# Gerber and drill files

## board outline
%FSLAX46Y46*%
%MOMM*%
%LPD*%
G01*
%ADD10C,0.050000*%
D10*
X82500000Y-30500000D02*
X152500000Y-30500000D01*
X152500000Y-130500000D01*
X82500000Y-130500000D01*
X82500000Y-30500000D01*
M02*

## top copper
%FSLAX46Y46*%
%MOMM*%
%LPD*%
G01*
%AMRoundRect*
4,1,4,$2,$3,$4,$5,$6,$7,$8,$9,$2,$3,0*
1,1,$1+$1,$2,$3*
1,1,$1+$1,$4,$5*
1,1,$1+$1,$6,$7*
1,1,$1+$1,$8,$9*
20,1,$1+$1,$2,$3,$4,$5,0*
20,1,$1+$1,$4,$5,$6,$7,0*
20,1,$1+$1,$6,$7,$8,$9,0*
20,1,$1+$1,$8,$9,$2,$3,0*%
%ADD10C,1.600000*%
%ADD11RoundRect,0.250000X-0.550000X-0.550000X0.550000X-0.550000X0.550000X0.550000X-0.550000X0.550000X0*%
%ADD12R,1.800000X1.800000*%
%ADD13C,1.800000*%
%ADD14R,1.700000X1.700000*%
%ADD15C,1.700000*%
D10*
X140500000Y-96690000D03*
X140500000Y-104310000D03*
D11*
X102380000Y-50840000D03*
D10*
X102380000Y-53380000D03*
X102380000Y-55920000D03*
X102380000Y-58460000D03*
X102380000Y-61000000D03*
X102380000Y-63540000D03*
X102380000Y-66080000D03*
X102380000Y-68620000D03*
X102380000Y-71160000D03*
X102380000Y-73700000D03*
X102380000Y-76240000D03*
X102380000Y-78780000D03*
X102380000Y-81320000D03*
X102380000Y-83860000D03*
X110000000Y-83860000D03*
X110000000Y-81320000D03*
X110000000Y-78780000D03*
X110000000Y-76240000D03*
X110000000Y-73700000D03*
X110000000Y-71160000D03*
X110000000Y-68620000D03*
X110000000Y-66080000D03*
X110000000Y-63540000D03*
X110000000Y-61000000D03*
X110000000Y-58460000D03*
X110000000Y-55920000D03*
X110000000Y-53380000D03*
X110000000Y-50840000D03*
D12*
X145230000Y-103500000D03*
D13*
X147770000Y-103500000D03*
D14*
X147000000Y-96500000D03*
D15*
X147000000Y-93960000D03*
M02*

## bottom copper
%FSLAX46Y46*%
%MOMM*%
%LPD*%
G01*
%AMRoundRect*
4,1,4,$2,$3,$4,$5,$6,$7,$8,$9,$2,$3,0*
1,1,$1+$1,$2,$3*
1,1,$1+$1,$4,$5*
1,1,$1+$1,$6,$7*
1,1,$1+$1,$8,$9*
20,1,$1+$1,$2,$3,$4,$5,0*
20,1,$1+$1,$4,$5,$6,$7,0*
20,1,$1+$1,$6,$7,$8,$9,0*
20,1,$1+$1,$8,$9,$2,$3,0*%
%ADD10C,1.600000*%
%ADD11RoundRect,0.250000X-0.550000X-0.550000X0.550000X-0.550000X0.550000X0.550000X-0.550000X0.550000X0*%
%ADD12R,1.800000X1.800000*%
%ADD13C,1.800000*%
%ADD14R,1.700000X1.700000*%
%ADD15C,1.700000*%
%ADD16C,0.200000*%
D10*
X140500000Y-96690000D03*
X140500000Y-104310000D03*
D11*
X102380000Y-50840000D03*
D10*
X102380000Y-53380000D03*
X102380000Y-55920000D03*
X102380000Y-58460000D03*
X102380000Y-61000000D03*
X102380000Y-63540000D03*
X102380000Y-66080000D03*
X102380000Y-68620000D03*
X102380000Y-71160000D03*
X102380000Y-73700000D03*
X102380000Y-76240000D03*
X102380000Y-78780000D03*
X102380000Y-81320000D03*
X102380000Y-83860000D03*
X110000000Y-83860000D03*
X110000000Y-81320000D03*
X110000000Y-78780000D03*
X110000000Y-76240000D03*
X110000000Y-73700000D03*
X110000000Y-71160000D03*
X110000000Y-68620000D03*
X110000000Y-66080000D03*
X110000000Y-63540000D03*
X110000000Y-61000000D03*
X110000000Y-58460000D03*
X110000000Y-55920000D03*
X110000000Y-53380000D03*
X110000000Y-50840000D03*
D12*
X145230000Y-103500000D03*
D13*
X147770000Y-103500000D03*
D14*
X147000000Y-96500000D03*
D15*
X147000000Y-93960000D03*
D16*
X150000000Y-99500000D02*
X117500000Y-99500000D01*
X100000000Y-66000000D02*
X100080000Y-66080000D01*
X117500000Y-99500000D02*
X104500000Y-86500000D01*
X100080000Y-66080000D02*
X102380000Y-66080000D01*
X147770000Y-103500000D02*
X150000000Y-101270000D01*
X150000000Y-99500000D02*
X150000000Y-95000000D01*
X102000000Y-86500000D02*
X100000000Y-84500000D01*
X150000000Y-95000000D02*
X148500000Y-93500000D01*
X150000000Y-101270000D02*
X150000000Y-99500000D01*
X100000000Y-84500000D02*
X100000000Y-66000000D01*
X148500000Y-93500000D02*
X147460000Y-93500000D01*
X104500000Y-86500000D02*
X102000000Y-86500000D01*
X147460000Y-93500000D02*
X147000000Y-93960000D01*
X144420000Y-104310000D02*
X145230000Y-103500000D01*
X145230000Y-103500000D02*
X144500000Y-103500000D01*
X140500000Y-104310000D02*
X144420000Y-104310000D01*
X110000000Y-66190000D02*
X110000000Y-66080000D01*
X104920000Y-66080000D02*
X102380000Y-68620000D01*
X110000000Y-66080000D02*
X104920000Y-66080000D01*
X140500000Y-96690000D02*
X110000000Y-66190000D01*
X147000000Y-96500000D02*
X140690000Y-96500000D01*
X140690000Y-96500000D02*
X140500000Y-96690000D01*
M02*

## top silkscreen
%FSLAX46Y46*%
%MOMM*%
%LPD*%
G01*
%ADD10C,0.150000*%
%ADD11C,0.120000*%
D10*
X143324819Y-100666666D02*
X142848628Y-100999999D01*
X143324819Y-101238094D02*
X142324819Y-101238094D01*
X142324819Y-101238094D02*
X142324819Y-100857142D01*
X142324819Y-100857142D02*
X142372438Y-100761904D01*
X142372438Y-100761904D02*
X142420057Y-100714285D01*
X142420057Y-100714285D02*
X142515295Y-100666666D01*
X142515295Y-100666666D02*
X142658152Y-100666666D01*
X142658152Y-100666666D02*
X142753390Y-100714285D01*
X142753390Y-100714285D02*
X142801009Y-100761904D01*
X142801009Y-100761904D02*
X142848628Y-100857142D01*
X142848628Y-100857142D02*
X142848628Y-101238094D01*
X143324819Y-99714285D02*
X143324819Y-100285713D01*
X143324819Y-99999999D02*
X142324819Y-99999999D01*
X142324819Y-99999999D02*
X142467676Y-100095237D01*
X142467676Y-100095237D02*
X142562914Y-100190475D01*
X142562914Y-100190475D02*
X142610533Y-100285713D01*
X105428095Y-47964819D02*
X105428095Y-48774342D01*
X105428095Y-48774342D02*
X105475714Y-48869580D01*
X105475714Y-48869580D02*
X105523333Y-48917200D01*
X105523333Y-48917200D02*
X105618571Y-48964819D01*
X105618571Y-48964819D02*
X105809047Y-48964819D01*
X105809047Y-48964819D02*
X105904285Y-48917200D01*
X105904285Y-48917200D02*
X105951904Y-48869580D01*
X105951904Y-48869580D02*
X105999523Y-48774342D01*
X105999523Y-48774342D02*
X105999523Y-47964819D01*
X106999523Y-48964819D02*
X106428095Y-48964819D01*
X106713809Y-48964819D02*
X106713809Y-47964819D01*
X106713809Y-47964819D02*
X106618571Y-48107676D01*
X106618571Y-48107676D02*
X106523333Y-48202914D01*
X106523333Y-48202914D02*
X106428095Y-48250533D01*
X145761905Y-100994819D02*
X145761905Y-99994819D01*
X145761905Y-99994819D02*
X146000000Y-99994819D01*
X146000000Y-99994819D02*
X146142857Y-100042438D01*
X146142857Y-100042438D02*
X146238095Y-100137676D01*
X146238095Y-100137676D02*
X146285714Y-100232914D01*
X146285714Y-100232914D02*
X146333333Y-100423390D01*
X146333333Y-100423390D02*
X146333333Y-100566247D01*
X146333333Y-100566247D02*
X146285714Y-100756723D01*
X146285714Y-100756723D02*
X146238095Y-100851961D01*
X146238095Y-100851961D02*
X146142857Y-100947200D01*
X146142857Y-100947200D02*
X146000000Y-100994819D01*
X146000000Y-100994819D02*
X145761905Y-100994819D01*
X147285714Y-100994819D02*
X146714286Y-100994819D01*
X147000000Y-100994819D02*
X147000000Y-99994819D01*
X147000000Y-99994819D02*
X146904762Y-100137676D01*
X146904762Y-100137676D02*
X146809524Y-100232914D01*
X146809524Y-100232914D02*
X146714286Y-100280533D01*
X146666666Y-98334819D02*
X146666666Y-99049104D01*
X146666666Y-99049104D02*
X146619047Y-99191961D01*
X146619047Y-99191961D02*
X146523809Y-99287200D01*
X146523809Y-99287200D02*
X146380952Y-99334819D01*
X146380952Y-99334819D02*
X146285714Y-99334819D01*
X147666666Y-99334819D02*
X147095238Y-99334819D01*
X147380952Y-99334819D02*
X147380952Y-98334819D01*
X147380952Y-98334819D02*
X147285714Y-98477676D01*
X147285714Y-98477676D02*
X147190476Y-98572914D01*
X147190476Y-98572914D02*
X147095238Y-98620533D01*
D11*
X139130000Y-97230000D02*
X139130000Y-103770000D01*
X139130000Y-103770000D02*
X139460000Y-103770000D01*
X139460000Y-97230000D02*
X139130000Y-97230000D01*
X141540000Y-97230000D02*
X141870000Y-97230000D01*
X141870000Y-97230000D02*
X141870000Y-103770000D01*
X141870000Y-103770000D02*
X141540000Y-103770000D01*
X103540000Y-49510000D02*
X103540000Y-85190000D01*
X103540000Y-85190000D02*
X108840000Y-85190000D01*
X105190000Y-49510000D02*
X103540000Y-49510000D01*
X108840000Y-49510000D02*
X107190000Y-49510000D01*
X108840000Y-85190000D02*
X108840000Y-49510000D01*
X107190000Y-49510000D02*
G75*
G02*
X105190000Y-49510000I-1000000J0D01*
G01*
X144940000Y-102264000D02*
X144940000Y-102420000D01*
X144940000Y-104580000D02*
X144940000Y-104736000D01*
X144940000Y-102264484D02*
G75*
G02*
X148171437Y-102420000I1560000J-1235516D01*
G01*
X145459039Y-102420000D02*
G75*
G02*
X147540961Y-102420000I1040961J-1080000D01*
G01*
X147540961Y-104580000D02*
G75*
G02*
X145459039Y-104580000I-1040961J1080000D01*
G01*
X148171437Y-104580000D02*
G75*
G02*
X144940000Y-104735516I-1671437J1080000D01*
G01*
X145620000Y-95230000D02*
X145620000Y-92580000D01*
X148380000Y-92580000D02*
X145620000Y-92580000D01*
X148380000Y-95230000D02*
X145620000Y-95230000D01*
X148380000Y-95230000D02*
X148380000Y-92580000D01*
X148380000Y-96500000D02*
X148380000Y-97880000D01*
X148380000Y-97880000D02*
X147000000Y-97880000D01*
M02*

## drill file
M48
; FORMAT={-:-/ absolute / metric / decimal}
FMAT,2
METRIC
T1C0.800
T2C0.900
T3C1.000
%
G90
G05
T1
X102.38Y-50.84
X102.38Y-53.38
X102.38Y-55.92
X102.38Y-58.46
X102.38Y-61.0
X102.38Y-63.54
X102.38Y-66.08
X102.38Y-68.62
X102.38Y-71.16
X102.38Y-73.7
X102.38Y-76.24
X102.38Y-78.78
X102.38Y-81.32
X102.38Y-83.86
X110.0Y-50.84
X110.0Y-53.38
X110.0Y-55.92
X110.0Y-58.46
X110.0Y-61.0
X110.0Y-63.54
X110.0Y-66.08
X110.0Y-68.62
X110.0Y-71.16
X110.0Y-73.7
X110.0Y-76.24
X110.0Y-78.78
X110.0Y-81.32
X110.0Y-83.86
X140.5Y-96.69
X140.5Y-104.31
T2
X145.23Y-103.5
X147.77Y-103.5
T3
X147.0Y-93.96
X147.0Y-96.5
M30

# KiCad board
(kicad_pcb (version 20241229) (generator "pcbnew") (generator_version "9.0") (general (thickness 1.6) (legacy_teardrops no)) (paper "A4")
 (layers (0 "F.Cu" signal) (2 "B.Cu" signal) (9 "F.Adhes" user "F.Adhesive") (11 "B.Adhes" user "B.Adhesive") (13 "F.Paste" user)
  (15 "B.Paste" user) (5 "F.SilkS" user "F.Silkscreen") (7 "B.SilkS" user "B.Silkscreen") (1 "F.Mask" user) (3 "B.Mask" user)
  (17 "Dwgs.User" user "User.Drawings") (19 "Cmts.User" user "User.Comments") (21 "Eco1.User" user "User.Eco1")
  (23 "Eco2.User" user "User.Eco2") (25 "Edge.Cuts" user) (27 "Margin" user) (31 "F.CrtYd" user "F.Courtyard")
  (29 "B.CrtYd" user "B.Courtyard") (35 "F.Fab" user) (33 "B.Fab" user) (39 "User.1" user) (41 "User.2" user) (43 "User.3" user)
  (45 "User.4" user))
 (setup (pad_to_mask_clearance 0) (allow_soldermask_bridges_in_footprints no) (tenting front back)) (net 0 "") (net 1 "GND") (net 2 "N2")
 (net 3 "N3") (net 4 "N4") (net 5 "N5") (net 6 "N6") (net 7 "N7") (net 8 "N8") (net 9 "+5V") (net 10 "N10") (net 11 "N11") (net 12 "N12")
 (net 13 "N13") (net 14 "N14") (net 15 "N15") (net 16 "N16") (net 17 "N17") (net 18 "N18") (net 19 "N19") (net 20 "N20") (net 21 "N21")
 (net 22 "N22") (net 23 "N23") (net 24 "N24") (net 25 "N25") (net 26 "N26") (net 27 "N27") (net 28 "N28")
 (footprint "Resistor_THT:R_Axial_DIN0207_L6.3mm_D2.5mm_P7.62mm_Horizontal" (layer "F.Cu") (at 140.5 96.69 -90)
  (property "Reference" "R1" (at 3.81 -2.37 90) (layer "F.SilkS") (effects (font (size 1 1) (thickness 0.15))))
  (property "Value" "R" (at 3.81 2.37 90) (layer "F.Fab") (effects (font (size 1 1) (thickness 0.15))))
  (fp_line (start 0.54 1.37) (end 7.08 1.37) (stroke (width 0.12) (type solid)) (layer "F.SilkS"))
  (fp_line (start 7.08 1.37) (end 7.08 1.04) (stroke (width 0.12) (type solid)) (layer "F.SilkS"))
  (fp_line (start 0.54 1.04) (end 0.54 1.37) (stroke (width 0.12) (type solid)) (layer "F.SilkS"))
  (fp_line (start 0.54 -1.04) (end 0.54 -1.37) (stroke (width 0.12) (type solid)) (layer "F.SilkS"))
  (fp_line (start 0.54 -1.37) (end 7.08 -1.37) (stroke (width 0.12) (type solid)) (layer "F.SilkS"))
  (fp_line (start 7.08 -1.37) (end 7.08 -1.04) (stroke (width 0.12) (type solid)) (layer "F.SilkS"))
  (pad "1" thru_hole circle (at 0 0 270) (size 1.6 1.6) (drill 0.8) (layers "*.Cu" "*.Mask") (remove_unused_layers no) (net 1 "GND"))
  (pad "2" thru_hole circle (at 7.62 0 270) (size 1.6 1.6) (drill 0.8) (layers "*.Cu" "*.Mask") (remove_unused_layers no) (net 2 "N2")))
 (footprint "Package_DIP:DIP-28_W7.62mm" (layer "F.Cu") (at 102.38 50.84)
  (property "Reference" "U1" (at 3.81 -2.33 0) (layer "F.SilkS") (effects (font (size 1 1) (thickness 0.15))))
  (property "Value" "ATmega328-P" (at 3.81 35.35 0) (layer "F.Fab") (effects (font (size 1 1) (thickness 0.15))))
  (fp_line (start 1.16 -1.33) (end 1.16 34.35) (stroke (width 0.12) (type solid)) (layer "F.SilkS"))
  (fp_line (start 1.16 34.35) (end 6.46 34.35) (stroke (width 0.12) (type solid)) (layer "F.SilkS"))
  (fp_line (start 2.81 -1.33) (end 1.16 -1.33) (stroke (width 0.12) (type solid)) (layer "F.SilkS"))
  (fp_line (start 6.46 -1.33) (end 4.81 -1.33) (stroke (width 0.12) (type solid)) (layer "F.SilkS"))
  (fp_line (start 6.46 34.35) (end 6.46 -1.33) (stroke (width 0.12) (type solid)) (layer "F.SilkS"))
  (fp_arc (start 4.81 -1.33) (mid 3.81 -0.33) (end 2.81 -1.33) (stroke (width 0.12) (type solid)) (layer "F.SilkS"))
  (pad "1" thru_hole roundrect (at 0 0) (size 1.6 1.6) (drill 0.8) (layers "*.Cu" "*.Mask") (remove_unused_layers no)
   (roundrect_rratio 0.15625) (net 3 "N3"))
  (pad "2" thru_hole circle (at 0 2.54) (size 1.6 1.6) (drill 0.8) (layers "*.Cu" "*.Mask") (remove_unused_layers no) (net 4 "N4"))
  (pad "3" thru_hole circle (at 0 5.08) (size 1.6 1.6) (drill 0.8) (layers "*.Cu" "*.Mask") (remove_unused_layers no) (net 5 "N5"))
  (pad "4" thru_hole circle (at 0 7.62) (size 1.6 1.6) (drill 0.8) (layers "*.Cu" "*.Mask") (remove_unused_layers no) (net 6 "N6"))
  (pad "5" thru_hole circle (at 0 10.16) (size 1.6 1.6) (drill 0.8) (layers "*.Cu" "*.Mask") (remove_unused_layers no) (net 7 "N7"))
  (pad "6" thru_hole circle (at 0 12.7) (size 1.6 1.6) (drill 0.8) (layers "*.Cu" "*.Mask") (remove_unused_layers no) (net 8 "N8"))
  (pad "7" thru_hole circle (at 0 15.24) (size 1.6 1.6) (drill 0.8) (layers "*.Cu" "*.Mask") (remove_unused_layers no) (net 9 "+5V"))
  (pad "8" thru_hole circle (at 0 17.78) (size 1.6 1.6) (drill 0.8) (layers "*.Cu" "*.Mask") (remove_unused_layers no) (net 1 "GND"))
  (pad "9" thru_hole circle (at 0 20.32) (size 1.6 1.6) (drill 0.8) (layers "*.Cu" "*.Mask") (remove_unused_layers no) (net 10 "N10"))
  (pad "10" thru_hole circle (at 0 22.86) (size 1.6 1.6) (drill 0.8) (layers "*.Cu" "*.Mask") (remove_unused_layers no) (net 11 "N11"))
  (pad "11" thru_hole circle (at 0 25.4) (size 1.6 1.6) (drill 0.8) (layers "*.Cu" "*.Mask") (remove_unused_layers no) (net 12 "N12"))
  (pad "12" thru_hole circle (at 0 27.94) (size 1.6 1.6) (drill 0.8) (layers "*.Cu" "*.Mask") (remove_unused_layers no) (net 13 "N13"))
  (pad "13" thru_hole circle (at 0 30.48) (size 1.6 1.6) (drill 0.8) (layers "*.Cu" "*.Mask") (remove_unused_layers no) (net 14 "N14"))
  (pad "14" thru_hole circle (at 0 33.02) (size 1.6 1.6) (drill 0.8) (layers "*.Cu" "*.Mask") (remove_unused_layers no) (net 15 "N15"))
  (pad "15" thru_hole circle (at 7.62 33.02) (size 1.6 1.6) (drill 0.8) (layers "*.Cu" "*.Mask") (remove_unused_layers no) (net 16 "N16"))
  (pad "16" thru_hole circle (at 7.62 30.48) (size 1.6 1.6) (drill 0.8) (layers "*.Cu" "*.Mask") (remove_unused_layers no) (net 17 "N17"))
  (pad "17" thru_hole circle (at 7.62 27.94) (size 1.6 1.6) (drill 0.8) (layers "*.Cu" "*.Mask") (remove_unused_layers no) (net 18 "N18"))
  (pad "18" thru_hole circle (at 7.62 25.4) (size 1.6 1.6) (drill 0.8) (layers "*.Cu" "*.Mask") (remove_unused_layers no) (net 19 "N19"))
  (pad "19" thru_hole circle (at 7.62 22.86) (size 1.6 1.6) (drill 0.8) (layers "*.Cu" "*.Mask") (remove_unused_layers no) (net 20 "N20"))
  (pad "20" thru_hole circle (at 7.62 20.32) (size 1.6 1.6) (drill 0.8) (layers "*.Cu" "*.Mask") (remove_unused_layers no) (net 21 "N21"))
  (pad "21" thru_hole circle (at 7.62 17.78) (size 1.6 1.6) (drill 0.8) (layers "*.Cu" "*.Mask") (remove_unused_layers no) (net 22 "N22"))
  (pad "22" thru_hole circle (at 7.62 15.24) (size 1.6 1.6) (drill 0.8) (layers "*.Cu" "*.Mask") (remove_unused_layers no) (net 1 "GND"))
  (pad "23" thru_hole circle (at 7.62 12.7) (size 1.6 1.6) (drill 0.8) (layers "*.Cu" "*.Mask") (remove_unused_layers no) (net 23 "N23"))
  (pad "24" thru_hole circle (at 7.62 10.16) (size 1.6 1.6) (drill 0.8) (layers "*.Cu" "*.Mask") (remove_unused_layers no) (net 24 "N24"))
  (pad "25" thru_hole circle (at 7.62 7.62) (size 1.6 1.6) (drill 0.8) (layers "*.Cu" "*.Mask") (remove_unused_layers no) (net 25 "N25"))
  (pad "26" thru_hole circle (at 7.62 5.08) (size 1.6 1.6) (drill 0.8) (layers "*.Cu" "*.Mask") (remove_unused_layers no) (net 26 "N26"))
  (pad "27" thru_hole circle (at 7.62 2.54) (size 1.6 1.6) (drill 0.8) (layers "*.Cu" "*.Mask") (remove_unused_layers no) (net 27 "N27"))
  (pad "28" thru_hole circle (at 7.62 0) (size 1.6 1.6) (drill 0.8) (layers "*.Cu" "*.Mask") (remove_unused_layers no) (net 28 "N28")))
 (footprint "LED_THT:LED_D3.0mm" (layer "F.Cu") (at 145.23 103.5)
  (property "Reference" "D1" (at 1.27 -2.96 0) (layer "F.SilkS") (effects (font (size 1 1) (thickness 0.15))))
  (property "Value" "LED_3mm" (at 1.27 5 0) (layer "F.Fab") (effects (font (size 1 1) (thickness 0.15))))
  (fp_line (start -0.29 -1.236) (end -0.29 -1.08) (stroke (width 0.12) (type solid)) (layer "F.SilkS"))
  (fp_line (start -0.29 1.08) (end -0.29 1.236) (stroke (width 0.12) (type solid)) (layer "F.SilkS"))
  (fp_arc (start -0.29 -1.235516) (mid 1.36566 -1.987699) (end 2.941437 -1.08) (stroke (width 0.12) (type solid)) (layer "F.SilkS"))
  (fp_arc (start 0.229039 -1.08) (mid 1.27 -1.5) (end 2.310961 -1.08) (stroke (width 0.12) (type solid)) (layer "F.SilkS"))
  (fp_arc (start 2.310961 1.08) (mid 1.27 1.5) (end 0.229039 1.08) (stroke (width 0.12) (type solid)) (layer "F.SilkS"))
  (fp_arc (start 2.941437 1.08) (mid 1.36566 1.987699) (end -0.29 1.235516) (stroke (width 0.12) (type solid)) (layer "F.SilkS"))
  (pad "1" thru_hole rect (at 0 0) (size 1.8 1.8) (drill 0.9) (layers "*.Cu" "*.Mask") (remove_unused_layers no) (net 2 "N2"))
  (pad "2" thru_hole circle (at 2.54 0) (size 1.8 1.8) (drill 0.9) (layers "*.Cu" "*.Mask") (remove_unused_layers no) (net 9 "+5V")))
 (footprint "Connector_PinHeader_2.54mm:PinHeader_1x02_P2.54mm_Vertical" (layer "F.Cu") (at 147 96.5 180)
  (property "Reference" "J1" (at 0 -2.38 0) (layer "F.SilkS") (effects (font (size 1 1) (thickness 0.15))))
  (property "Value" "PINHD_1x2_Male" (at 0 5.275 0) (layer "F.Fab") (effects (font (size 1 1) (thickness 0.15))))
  (fp_line (start 1.38 1.27) (end 1.38 3.92) (stroke (width 0.12) (type solid)) (layer "F.SilkS"))
  (fp_line (start -1.38 3.92) (end 1.38 3.92) (stroke (width 0.12) (type solid)) (layer "F.SilkS"))
  (fp_line (start -1.38 1.27) (end 1.38 1.27) (stroke (width 0.12) (type solid)) (layer "F.SilkS"))
  (fp_line (start -1.38 1.27) (end -1.38 3.92) (stroke (width 0.12) (type solid)) (layer "F.SilkS"))
  (fp_line (start -1.38 0) (end -1.38 -1.38) (stroke (width 0.12) (type solid)) (layer "F.SilkS"))
  (fp_line (start -1.38 -1.38) (end 0 -1.38) (stroke (width 0.12) (type solid)) (layer "F.SilkS"))
  (pad "1" thru_hole rect (at 0 0 180) (size 1.7 1.7) (drill 1) (layers "*.Cu" "*.Mask") (remove_unused_layers no) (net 1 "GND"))
  (pad "2" thru_hole circle (at 0 2.54 180) (size 1.7 1.7) (drill 1) (layers "*.Cu" "*.Mask") (remove_unused_layers no) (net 9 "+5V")))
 (gr_rect (start 82.5 30.5) (end 152.5 130.5) (stroke (width 0.05) (type default)) (fill no) (layer "Edge.Cuts"))
 (segment (start 150 99.5) (end 117.5 99.5) (width 0.2) (layer "B.Cu") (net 9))
 (segment (start 100 66) (end 100.08 66.08) (width 0.2) (layer "B.Cu") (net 9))
 (segment (start 117.5 99.5) (end 104.5 86.5) (width 0.2) (layer "B.Cu") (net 9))
 (segment (start 100.08 66.08) (end 102.38 66.08) (width 0.2) (layer "B.Cu") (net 9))
 (segment (start 147.77 103.5) (end 150 101.27) (width 0.2) (layer "B.Cu") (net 9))
 (segment (start 150 99.5) (end 150 95) (width 0.2) (layer "B.Cu") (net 9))
 (segment (start 102 86.5) (end 100 84.5) (width 0.2) (layer "B.Cu") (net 9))
 (segment (start 150 95) (end 148.5 93.5) (width 0.2) (layer "B.Cu") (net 9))
 (segment (start 150 101.27) (end 150 99.5) (width 0.2) (layer "B.Cu") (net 9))
 (segment (start 100 84.5) (end 100 66) (width 0.2) (layer "B.Cu") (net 9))
 (segment (start 148.5 93.5) (end 147.46 93.5) (width 0.2) (layer "B.Cu") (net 9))
 (segment (start 104.5 86.5) (end 102 86.5) (width 0.2) (layer "B.Cu") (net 9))
 (segment (start 147.46 93.5) (end 147 93.96) (width 0.2) (layer "B.Cu") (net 9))
 (segment (start 144.42 104.31) (end 145.23 103.5) (width 0.2) (layer "B.Cu") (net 2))
 (segment (start 145.23 103.5) (end 144.5 103.5) (width 0.2) (layer "B.Cu") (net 2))
 (segment (start 140.5 104.31) (end 144.42 104.31) (width 0.2) (layer "B.Cu") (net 2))
 (segment (start 110 66.19) (end 110 66.08) (width 0.2) (layer "B.Cu") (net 1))
 (segment (start 104.92 66.08) (end 102.38 68.62) (width 0.2) (layer "B.Cu") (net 1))
 (segment (start 110 66.08) (end 104.92 66.08) (width 0.2) (layer "B.Cu") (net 1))
 (segment (start 140.5 96.69) (end 110 66.19) (width 0.2) (layer "B.Cu") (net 1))
 (segment (start 147 96.5) (end 140.69 96.5) (width 0.2) (layer "B.Cu") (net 1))
 (segment (start 140.69 96.5) (end 140.5 96.69) (width 0.2) (layer "B.Cu") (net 1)))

